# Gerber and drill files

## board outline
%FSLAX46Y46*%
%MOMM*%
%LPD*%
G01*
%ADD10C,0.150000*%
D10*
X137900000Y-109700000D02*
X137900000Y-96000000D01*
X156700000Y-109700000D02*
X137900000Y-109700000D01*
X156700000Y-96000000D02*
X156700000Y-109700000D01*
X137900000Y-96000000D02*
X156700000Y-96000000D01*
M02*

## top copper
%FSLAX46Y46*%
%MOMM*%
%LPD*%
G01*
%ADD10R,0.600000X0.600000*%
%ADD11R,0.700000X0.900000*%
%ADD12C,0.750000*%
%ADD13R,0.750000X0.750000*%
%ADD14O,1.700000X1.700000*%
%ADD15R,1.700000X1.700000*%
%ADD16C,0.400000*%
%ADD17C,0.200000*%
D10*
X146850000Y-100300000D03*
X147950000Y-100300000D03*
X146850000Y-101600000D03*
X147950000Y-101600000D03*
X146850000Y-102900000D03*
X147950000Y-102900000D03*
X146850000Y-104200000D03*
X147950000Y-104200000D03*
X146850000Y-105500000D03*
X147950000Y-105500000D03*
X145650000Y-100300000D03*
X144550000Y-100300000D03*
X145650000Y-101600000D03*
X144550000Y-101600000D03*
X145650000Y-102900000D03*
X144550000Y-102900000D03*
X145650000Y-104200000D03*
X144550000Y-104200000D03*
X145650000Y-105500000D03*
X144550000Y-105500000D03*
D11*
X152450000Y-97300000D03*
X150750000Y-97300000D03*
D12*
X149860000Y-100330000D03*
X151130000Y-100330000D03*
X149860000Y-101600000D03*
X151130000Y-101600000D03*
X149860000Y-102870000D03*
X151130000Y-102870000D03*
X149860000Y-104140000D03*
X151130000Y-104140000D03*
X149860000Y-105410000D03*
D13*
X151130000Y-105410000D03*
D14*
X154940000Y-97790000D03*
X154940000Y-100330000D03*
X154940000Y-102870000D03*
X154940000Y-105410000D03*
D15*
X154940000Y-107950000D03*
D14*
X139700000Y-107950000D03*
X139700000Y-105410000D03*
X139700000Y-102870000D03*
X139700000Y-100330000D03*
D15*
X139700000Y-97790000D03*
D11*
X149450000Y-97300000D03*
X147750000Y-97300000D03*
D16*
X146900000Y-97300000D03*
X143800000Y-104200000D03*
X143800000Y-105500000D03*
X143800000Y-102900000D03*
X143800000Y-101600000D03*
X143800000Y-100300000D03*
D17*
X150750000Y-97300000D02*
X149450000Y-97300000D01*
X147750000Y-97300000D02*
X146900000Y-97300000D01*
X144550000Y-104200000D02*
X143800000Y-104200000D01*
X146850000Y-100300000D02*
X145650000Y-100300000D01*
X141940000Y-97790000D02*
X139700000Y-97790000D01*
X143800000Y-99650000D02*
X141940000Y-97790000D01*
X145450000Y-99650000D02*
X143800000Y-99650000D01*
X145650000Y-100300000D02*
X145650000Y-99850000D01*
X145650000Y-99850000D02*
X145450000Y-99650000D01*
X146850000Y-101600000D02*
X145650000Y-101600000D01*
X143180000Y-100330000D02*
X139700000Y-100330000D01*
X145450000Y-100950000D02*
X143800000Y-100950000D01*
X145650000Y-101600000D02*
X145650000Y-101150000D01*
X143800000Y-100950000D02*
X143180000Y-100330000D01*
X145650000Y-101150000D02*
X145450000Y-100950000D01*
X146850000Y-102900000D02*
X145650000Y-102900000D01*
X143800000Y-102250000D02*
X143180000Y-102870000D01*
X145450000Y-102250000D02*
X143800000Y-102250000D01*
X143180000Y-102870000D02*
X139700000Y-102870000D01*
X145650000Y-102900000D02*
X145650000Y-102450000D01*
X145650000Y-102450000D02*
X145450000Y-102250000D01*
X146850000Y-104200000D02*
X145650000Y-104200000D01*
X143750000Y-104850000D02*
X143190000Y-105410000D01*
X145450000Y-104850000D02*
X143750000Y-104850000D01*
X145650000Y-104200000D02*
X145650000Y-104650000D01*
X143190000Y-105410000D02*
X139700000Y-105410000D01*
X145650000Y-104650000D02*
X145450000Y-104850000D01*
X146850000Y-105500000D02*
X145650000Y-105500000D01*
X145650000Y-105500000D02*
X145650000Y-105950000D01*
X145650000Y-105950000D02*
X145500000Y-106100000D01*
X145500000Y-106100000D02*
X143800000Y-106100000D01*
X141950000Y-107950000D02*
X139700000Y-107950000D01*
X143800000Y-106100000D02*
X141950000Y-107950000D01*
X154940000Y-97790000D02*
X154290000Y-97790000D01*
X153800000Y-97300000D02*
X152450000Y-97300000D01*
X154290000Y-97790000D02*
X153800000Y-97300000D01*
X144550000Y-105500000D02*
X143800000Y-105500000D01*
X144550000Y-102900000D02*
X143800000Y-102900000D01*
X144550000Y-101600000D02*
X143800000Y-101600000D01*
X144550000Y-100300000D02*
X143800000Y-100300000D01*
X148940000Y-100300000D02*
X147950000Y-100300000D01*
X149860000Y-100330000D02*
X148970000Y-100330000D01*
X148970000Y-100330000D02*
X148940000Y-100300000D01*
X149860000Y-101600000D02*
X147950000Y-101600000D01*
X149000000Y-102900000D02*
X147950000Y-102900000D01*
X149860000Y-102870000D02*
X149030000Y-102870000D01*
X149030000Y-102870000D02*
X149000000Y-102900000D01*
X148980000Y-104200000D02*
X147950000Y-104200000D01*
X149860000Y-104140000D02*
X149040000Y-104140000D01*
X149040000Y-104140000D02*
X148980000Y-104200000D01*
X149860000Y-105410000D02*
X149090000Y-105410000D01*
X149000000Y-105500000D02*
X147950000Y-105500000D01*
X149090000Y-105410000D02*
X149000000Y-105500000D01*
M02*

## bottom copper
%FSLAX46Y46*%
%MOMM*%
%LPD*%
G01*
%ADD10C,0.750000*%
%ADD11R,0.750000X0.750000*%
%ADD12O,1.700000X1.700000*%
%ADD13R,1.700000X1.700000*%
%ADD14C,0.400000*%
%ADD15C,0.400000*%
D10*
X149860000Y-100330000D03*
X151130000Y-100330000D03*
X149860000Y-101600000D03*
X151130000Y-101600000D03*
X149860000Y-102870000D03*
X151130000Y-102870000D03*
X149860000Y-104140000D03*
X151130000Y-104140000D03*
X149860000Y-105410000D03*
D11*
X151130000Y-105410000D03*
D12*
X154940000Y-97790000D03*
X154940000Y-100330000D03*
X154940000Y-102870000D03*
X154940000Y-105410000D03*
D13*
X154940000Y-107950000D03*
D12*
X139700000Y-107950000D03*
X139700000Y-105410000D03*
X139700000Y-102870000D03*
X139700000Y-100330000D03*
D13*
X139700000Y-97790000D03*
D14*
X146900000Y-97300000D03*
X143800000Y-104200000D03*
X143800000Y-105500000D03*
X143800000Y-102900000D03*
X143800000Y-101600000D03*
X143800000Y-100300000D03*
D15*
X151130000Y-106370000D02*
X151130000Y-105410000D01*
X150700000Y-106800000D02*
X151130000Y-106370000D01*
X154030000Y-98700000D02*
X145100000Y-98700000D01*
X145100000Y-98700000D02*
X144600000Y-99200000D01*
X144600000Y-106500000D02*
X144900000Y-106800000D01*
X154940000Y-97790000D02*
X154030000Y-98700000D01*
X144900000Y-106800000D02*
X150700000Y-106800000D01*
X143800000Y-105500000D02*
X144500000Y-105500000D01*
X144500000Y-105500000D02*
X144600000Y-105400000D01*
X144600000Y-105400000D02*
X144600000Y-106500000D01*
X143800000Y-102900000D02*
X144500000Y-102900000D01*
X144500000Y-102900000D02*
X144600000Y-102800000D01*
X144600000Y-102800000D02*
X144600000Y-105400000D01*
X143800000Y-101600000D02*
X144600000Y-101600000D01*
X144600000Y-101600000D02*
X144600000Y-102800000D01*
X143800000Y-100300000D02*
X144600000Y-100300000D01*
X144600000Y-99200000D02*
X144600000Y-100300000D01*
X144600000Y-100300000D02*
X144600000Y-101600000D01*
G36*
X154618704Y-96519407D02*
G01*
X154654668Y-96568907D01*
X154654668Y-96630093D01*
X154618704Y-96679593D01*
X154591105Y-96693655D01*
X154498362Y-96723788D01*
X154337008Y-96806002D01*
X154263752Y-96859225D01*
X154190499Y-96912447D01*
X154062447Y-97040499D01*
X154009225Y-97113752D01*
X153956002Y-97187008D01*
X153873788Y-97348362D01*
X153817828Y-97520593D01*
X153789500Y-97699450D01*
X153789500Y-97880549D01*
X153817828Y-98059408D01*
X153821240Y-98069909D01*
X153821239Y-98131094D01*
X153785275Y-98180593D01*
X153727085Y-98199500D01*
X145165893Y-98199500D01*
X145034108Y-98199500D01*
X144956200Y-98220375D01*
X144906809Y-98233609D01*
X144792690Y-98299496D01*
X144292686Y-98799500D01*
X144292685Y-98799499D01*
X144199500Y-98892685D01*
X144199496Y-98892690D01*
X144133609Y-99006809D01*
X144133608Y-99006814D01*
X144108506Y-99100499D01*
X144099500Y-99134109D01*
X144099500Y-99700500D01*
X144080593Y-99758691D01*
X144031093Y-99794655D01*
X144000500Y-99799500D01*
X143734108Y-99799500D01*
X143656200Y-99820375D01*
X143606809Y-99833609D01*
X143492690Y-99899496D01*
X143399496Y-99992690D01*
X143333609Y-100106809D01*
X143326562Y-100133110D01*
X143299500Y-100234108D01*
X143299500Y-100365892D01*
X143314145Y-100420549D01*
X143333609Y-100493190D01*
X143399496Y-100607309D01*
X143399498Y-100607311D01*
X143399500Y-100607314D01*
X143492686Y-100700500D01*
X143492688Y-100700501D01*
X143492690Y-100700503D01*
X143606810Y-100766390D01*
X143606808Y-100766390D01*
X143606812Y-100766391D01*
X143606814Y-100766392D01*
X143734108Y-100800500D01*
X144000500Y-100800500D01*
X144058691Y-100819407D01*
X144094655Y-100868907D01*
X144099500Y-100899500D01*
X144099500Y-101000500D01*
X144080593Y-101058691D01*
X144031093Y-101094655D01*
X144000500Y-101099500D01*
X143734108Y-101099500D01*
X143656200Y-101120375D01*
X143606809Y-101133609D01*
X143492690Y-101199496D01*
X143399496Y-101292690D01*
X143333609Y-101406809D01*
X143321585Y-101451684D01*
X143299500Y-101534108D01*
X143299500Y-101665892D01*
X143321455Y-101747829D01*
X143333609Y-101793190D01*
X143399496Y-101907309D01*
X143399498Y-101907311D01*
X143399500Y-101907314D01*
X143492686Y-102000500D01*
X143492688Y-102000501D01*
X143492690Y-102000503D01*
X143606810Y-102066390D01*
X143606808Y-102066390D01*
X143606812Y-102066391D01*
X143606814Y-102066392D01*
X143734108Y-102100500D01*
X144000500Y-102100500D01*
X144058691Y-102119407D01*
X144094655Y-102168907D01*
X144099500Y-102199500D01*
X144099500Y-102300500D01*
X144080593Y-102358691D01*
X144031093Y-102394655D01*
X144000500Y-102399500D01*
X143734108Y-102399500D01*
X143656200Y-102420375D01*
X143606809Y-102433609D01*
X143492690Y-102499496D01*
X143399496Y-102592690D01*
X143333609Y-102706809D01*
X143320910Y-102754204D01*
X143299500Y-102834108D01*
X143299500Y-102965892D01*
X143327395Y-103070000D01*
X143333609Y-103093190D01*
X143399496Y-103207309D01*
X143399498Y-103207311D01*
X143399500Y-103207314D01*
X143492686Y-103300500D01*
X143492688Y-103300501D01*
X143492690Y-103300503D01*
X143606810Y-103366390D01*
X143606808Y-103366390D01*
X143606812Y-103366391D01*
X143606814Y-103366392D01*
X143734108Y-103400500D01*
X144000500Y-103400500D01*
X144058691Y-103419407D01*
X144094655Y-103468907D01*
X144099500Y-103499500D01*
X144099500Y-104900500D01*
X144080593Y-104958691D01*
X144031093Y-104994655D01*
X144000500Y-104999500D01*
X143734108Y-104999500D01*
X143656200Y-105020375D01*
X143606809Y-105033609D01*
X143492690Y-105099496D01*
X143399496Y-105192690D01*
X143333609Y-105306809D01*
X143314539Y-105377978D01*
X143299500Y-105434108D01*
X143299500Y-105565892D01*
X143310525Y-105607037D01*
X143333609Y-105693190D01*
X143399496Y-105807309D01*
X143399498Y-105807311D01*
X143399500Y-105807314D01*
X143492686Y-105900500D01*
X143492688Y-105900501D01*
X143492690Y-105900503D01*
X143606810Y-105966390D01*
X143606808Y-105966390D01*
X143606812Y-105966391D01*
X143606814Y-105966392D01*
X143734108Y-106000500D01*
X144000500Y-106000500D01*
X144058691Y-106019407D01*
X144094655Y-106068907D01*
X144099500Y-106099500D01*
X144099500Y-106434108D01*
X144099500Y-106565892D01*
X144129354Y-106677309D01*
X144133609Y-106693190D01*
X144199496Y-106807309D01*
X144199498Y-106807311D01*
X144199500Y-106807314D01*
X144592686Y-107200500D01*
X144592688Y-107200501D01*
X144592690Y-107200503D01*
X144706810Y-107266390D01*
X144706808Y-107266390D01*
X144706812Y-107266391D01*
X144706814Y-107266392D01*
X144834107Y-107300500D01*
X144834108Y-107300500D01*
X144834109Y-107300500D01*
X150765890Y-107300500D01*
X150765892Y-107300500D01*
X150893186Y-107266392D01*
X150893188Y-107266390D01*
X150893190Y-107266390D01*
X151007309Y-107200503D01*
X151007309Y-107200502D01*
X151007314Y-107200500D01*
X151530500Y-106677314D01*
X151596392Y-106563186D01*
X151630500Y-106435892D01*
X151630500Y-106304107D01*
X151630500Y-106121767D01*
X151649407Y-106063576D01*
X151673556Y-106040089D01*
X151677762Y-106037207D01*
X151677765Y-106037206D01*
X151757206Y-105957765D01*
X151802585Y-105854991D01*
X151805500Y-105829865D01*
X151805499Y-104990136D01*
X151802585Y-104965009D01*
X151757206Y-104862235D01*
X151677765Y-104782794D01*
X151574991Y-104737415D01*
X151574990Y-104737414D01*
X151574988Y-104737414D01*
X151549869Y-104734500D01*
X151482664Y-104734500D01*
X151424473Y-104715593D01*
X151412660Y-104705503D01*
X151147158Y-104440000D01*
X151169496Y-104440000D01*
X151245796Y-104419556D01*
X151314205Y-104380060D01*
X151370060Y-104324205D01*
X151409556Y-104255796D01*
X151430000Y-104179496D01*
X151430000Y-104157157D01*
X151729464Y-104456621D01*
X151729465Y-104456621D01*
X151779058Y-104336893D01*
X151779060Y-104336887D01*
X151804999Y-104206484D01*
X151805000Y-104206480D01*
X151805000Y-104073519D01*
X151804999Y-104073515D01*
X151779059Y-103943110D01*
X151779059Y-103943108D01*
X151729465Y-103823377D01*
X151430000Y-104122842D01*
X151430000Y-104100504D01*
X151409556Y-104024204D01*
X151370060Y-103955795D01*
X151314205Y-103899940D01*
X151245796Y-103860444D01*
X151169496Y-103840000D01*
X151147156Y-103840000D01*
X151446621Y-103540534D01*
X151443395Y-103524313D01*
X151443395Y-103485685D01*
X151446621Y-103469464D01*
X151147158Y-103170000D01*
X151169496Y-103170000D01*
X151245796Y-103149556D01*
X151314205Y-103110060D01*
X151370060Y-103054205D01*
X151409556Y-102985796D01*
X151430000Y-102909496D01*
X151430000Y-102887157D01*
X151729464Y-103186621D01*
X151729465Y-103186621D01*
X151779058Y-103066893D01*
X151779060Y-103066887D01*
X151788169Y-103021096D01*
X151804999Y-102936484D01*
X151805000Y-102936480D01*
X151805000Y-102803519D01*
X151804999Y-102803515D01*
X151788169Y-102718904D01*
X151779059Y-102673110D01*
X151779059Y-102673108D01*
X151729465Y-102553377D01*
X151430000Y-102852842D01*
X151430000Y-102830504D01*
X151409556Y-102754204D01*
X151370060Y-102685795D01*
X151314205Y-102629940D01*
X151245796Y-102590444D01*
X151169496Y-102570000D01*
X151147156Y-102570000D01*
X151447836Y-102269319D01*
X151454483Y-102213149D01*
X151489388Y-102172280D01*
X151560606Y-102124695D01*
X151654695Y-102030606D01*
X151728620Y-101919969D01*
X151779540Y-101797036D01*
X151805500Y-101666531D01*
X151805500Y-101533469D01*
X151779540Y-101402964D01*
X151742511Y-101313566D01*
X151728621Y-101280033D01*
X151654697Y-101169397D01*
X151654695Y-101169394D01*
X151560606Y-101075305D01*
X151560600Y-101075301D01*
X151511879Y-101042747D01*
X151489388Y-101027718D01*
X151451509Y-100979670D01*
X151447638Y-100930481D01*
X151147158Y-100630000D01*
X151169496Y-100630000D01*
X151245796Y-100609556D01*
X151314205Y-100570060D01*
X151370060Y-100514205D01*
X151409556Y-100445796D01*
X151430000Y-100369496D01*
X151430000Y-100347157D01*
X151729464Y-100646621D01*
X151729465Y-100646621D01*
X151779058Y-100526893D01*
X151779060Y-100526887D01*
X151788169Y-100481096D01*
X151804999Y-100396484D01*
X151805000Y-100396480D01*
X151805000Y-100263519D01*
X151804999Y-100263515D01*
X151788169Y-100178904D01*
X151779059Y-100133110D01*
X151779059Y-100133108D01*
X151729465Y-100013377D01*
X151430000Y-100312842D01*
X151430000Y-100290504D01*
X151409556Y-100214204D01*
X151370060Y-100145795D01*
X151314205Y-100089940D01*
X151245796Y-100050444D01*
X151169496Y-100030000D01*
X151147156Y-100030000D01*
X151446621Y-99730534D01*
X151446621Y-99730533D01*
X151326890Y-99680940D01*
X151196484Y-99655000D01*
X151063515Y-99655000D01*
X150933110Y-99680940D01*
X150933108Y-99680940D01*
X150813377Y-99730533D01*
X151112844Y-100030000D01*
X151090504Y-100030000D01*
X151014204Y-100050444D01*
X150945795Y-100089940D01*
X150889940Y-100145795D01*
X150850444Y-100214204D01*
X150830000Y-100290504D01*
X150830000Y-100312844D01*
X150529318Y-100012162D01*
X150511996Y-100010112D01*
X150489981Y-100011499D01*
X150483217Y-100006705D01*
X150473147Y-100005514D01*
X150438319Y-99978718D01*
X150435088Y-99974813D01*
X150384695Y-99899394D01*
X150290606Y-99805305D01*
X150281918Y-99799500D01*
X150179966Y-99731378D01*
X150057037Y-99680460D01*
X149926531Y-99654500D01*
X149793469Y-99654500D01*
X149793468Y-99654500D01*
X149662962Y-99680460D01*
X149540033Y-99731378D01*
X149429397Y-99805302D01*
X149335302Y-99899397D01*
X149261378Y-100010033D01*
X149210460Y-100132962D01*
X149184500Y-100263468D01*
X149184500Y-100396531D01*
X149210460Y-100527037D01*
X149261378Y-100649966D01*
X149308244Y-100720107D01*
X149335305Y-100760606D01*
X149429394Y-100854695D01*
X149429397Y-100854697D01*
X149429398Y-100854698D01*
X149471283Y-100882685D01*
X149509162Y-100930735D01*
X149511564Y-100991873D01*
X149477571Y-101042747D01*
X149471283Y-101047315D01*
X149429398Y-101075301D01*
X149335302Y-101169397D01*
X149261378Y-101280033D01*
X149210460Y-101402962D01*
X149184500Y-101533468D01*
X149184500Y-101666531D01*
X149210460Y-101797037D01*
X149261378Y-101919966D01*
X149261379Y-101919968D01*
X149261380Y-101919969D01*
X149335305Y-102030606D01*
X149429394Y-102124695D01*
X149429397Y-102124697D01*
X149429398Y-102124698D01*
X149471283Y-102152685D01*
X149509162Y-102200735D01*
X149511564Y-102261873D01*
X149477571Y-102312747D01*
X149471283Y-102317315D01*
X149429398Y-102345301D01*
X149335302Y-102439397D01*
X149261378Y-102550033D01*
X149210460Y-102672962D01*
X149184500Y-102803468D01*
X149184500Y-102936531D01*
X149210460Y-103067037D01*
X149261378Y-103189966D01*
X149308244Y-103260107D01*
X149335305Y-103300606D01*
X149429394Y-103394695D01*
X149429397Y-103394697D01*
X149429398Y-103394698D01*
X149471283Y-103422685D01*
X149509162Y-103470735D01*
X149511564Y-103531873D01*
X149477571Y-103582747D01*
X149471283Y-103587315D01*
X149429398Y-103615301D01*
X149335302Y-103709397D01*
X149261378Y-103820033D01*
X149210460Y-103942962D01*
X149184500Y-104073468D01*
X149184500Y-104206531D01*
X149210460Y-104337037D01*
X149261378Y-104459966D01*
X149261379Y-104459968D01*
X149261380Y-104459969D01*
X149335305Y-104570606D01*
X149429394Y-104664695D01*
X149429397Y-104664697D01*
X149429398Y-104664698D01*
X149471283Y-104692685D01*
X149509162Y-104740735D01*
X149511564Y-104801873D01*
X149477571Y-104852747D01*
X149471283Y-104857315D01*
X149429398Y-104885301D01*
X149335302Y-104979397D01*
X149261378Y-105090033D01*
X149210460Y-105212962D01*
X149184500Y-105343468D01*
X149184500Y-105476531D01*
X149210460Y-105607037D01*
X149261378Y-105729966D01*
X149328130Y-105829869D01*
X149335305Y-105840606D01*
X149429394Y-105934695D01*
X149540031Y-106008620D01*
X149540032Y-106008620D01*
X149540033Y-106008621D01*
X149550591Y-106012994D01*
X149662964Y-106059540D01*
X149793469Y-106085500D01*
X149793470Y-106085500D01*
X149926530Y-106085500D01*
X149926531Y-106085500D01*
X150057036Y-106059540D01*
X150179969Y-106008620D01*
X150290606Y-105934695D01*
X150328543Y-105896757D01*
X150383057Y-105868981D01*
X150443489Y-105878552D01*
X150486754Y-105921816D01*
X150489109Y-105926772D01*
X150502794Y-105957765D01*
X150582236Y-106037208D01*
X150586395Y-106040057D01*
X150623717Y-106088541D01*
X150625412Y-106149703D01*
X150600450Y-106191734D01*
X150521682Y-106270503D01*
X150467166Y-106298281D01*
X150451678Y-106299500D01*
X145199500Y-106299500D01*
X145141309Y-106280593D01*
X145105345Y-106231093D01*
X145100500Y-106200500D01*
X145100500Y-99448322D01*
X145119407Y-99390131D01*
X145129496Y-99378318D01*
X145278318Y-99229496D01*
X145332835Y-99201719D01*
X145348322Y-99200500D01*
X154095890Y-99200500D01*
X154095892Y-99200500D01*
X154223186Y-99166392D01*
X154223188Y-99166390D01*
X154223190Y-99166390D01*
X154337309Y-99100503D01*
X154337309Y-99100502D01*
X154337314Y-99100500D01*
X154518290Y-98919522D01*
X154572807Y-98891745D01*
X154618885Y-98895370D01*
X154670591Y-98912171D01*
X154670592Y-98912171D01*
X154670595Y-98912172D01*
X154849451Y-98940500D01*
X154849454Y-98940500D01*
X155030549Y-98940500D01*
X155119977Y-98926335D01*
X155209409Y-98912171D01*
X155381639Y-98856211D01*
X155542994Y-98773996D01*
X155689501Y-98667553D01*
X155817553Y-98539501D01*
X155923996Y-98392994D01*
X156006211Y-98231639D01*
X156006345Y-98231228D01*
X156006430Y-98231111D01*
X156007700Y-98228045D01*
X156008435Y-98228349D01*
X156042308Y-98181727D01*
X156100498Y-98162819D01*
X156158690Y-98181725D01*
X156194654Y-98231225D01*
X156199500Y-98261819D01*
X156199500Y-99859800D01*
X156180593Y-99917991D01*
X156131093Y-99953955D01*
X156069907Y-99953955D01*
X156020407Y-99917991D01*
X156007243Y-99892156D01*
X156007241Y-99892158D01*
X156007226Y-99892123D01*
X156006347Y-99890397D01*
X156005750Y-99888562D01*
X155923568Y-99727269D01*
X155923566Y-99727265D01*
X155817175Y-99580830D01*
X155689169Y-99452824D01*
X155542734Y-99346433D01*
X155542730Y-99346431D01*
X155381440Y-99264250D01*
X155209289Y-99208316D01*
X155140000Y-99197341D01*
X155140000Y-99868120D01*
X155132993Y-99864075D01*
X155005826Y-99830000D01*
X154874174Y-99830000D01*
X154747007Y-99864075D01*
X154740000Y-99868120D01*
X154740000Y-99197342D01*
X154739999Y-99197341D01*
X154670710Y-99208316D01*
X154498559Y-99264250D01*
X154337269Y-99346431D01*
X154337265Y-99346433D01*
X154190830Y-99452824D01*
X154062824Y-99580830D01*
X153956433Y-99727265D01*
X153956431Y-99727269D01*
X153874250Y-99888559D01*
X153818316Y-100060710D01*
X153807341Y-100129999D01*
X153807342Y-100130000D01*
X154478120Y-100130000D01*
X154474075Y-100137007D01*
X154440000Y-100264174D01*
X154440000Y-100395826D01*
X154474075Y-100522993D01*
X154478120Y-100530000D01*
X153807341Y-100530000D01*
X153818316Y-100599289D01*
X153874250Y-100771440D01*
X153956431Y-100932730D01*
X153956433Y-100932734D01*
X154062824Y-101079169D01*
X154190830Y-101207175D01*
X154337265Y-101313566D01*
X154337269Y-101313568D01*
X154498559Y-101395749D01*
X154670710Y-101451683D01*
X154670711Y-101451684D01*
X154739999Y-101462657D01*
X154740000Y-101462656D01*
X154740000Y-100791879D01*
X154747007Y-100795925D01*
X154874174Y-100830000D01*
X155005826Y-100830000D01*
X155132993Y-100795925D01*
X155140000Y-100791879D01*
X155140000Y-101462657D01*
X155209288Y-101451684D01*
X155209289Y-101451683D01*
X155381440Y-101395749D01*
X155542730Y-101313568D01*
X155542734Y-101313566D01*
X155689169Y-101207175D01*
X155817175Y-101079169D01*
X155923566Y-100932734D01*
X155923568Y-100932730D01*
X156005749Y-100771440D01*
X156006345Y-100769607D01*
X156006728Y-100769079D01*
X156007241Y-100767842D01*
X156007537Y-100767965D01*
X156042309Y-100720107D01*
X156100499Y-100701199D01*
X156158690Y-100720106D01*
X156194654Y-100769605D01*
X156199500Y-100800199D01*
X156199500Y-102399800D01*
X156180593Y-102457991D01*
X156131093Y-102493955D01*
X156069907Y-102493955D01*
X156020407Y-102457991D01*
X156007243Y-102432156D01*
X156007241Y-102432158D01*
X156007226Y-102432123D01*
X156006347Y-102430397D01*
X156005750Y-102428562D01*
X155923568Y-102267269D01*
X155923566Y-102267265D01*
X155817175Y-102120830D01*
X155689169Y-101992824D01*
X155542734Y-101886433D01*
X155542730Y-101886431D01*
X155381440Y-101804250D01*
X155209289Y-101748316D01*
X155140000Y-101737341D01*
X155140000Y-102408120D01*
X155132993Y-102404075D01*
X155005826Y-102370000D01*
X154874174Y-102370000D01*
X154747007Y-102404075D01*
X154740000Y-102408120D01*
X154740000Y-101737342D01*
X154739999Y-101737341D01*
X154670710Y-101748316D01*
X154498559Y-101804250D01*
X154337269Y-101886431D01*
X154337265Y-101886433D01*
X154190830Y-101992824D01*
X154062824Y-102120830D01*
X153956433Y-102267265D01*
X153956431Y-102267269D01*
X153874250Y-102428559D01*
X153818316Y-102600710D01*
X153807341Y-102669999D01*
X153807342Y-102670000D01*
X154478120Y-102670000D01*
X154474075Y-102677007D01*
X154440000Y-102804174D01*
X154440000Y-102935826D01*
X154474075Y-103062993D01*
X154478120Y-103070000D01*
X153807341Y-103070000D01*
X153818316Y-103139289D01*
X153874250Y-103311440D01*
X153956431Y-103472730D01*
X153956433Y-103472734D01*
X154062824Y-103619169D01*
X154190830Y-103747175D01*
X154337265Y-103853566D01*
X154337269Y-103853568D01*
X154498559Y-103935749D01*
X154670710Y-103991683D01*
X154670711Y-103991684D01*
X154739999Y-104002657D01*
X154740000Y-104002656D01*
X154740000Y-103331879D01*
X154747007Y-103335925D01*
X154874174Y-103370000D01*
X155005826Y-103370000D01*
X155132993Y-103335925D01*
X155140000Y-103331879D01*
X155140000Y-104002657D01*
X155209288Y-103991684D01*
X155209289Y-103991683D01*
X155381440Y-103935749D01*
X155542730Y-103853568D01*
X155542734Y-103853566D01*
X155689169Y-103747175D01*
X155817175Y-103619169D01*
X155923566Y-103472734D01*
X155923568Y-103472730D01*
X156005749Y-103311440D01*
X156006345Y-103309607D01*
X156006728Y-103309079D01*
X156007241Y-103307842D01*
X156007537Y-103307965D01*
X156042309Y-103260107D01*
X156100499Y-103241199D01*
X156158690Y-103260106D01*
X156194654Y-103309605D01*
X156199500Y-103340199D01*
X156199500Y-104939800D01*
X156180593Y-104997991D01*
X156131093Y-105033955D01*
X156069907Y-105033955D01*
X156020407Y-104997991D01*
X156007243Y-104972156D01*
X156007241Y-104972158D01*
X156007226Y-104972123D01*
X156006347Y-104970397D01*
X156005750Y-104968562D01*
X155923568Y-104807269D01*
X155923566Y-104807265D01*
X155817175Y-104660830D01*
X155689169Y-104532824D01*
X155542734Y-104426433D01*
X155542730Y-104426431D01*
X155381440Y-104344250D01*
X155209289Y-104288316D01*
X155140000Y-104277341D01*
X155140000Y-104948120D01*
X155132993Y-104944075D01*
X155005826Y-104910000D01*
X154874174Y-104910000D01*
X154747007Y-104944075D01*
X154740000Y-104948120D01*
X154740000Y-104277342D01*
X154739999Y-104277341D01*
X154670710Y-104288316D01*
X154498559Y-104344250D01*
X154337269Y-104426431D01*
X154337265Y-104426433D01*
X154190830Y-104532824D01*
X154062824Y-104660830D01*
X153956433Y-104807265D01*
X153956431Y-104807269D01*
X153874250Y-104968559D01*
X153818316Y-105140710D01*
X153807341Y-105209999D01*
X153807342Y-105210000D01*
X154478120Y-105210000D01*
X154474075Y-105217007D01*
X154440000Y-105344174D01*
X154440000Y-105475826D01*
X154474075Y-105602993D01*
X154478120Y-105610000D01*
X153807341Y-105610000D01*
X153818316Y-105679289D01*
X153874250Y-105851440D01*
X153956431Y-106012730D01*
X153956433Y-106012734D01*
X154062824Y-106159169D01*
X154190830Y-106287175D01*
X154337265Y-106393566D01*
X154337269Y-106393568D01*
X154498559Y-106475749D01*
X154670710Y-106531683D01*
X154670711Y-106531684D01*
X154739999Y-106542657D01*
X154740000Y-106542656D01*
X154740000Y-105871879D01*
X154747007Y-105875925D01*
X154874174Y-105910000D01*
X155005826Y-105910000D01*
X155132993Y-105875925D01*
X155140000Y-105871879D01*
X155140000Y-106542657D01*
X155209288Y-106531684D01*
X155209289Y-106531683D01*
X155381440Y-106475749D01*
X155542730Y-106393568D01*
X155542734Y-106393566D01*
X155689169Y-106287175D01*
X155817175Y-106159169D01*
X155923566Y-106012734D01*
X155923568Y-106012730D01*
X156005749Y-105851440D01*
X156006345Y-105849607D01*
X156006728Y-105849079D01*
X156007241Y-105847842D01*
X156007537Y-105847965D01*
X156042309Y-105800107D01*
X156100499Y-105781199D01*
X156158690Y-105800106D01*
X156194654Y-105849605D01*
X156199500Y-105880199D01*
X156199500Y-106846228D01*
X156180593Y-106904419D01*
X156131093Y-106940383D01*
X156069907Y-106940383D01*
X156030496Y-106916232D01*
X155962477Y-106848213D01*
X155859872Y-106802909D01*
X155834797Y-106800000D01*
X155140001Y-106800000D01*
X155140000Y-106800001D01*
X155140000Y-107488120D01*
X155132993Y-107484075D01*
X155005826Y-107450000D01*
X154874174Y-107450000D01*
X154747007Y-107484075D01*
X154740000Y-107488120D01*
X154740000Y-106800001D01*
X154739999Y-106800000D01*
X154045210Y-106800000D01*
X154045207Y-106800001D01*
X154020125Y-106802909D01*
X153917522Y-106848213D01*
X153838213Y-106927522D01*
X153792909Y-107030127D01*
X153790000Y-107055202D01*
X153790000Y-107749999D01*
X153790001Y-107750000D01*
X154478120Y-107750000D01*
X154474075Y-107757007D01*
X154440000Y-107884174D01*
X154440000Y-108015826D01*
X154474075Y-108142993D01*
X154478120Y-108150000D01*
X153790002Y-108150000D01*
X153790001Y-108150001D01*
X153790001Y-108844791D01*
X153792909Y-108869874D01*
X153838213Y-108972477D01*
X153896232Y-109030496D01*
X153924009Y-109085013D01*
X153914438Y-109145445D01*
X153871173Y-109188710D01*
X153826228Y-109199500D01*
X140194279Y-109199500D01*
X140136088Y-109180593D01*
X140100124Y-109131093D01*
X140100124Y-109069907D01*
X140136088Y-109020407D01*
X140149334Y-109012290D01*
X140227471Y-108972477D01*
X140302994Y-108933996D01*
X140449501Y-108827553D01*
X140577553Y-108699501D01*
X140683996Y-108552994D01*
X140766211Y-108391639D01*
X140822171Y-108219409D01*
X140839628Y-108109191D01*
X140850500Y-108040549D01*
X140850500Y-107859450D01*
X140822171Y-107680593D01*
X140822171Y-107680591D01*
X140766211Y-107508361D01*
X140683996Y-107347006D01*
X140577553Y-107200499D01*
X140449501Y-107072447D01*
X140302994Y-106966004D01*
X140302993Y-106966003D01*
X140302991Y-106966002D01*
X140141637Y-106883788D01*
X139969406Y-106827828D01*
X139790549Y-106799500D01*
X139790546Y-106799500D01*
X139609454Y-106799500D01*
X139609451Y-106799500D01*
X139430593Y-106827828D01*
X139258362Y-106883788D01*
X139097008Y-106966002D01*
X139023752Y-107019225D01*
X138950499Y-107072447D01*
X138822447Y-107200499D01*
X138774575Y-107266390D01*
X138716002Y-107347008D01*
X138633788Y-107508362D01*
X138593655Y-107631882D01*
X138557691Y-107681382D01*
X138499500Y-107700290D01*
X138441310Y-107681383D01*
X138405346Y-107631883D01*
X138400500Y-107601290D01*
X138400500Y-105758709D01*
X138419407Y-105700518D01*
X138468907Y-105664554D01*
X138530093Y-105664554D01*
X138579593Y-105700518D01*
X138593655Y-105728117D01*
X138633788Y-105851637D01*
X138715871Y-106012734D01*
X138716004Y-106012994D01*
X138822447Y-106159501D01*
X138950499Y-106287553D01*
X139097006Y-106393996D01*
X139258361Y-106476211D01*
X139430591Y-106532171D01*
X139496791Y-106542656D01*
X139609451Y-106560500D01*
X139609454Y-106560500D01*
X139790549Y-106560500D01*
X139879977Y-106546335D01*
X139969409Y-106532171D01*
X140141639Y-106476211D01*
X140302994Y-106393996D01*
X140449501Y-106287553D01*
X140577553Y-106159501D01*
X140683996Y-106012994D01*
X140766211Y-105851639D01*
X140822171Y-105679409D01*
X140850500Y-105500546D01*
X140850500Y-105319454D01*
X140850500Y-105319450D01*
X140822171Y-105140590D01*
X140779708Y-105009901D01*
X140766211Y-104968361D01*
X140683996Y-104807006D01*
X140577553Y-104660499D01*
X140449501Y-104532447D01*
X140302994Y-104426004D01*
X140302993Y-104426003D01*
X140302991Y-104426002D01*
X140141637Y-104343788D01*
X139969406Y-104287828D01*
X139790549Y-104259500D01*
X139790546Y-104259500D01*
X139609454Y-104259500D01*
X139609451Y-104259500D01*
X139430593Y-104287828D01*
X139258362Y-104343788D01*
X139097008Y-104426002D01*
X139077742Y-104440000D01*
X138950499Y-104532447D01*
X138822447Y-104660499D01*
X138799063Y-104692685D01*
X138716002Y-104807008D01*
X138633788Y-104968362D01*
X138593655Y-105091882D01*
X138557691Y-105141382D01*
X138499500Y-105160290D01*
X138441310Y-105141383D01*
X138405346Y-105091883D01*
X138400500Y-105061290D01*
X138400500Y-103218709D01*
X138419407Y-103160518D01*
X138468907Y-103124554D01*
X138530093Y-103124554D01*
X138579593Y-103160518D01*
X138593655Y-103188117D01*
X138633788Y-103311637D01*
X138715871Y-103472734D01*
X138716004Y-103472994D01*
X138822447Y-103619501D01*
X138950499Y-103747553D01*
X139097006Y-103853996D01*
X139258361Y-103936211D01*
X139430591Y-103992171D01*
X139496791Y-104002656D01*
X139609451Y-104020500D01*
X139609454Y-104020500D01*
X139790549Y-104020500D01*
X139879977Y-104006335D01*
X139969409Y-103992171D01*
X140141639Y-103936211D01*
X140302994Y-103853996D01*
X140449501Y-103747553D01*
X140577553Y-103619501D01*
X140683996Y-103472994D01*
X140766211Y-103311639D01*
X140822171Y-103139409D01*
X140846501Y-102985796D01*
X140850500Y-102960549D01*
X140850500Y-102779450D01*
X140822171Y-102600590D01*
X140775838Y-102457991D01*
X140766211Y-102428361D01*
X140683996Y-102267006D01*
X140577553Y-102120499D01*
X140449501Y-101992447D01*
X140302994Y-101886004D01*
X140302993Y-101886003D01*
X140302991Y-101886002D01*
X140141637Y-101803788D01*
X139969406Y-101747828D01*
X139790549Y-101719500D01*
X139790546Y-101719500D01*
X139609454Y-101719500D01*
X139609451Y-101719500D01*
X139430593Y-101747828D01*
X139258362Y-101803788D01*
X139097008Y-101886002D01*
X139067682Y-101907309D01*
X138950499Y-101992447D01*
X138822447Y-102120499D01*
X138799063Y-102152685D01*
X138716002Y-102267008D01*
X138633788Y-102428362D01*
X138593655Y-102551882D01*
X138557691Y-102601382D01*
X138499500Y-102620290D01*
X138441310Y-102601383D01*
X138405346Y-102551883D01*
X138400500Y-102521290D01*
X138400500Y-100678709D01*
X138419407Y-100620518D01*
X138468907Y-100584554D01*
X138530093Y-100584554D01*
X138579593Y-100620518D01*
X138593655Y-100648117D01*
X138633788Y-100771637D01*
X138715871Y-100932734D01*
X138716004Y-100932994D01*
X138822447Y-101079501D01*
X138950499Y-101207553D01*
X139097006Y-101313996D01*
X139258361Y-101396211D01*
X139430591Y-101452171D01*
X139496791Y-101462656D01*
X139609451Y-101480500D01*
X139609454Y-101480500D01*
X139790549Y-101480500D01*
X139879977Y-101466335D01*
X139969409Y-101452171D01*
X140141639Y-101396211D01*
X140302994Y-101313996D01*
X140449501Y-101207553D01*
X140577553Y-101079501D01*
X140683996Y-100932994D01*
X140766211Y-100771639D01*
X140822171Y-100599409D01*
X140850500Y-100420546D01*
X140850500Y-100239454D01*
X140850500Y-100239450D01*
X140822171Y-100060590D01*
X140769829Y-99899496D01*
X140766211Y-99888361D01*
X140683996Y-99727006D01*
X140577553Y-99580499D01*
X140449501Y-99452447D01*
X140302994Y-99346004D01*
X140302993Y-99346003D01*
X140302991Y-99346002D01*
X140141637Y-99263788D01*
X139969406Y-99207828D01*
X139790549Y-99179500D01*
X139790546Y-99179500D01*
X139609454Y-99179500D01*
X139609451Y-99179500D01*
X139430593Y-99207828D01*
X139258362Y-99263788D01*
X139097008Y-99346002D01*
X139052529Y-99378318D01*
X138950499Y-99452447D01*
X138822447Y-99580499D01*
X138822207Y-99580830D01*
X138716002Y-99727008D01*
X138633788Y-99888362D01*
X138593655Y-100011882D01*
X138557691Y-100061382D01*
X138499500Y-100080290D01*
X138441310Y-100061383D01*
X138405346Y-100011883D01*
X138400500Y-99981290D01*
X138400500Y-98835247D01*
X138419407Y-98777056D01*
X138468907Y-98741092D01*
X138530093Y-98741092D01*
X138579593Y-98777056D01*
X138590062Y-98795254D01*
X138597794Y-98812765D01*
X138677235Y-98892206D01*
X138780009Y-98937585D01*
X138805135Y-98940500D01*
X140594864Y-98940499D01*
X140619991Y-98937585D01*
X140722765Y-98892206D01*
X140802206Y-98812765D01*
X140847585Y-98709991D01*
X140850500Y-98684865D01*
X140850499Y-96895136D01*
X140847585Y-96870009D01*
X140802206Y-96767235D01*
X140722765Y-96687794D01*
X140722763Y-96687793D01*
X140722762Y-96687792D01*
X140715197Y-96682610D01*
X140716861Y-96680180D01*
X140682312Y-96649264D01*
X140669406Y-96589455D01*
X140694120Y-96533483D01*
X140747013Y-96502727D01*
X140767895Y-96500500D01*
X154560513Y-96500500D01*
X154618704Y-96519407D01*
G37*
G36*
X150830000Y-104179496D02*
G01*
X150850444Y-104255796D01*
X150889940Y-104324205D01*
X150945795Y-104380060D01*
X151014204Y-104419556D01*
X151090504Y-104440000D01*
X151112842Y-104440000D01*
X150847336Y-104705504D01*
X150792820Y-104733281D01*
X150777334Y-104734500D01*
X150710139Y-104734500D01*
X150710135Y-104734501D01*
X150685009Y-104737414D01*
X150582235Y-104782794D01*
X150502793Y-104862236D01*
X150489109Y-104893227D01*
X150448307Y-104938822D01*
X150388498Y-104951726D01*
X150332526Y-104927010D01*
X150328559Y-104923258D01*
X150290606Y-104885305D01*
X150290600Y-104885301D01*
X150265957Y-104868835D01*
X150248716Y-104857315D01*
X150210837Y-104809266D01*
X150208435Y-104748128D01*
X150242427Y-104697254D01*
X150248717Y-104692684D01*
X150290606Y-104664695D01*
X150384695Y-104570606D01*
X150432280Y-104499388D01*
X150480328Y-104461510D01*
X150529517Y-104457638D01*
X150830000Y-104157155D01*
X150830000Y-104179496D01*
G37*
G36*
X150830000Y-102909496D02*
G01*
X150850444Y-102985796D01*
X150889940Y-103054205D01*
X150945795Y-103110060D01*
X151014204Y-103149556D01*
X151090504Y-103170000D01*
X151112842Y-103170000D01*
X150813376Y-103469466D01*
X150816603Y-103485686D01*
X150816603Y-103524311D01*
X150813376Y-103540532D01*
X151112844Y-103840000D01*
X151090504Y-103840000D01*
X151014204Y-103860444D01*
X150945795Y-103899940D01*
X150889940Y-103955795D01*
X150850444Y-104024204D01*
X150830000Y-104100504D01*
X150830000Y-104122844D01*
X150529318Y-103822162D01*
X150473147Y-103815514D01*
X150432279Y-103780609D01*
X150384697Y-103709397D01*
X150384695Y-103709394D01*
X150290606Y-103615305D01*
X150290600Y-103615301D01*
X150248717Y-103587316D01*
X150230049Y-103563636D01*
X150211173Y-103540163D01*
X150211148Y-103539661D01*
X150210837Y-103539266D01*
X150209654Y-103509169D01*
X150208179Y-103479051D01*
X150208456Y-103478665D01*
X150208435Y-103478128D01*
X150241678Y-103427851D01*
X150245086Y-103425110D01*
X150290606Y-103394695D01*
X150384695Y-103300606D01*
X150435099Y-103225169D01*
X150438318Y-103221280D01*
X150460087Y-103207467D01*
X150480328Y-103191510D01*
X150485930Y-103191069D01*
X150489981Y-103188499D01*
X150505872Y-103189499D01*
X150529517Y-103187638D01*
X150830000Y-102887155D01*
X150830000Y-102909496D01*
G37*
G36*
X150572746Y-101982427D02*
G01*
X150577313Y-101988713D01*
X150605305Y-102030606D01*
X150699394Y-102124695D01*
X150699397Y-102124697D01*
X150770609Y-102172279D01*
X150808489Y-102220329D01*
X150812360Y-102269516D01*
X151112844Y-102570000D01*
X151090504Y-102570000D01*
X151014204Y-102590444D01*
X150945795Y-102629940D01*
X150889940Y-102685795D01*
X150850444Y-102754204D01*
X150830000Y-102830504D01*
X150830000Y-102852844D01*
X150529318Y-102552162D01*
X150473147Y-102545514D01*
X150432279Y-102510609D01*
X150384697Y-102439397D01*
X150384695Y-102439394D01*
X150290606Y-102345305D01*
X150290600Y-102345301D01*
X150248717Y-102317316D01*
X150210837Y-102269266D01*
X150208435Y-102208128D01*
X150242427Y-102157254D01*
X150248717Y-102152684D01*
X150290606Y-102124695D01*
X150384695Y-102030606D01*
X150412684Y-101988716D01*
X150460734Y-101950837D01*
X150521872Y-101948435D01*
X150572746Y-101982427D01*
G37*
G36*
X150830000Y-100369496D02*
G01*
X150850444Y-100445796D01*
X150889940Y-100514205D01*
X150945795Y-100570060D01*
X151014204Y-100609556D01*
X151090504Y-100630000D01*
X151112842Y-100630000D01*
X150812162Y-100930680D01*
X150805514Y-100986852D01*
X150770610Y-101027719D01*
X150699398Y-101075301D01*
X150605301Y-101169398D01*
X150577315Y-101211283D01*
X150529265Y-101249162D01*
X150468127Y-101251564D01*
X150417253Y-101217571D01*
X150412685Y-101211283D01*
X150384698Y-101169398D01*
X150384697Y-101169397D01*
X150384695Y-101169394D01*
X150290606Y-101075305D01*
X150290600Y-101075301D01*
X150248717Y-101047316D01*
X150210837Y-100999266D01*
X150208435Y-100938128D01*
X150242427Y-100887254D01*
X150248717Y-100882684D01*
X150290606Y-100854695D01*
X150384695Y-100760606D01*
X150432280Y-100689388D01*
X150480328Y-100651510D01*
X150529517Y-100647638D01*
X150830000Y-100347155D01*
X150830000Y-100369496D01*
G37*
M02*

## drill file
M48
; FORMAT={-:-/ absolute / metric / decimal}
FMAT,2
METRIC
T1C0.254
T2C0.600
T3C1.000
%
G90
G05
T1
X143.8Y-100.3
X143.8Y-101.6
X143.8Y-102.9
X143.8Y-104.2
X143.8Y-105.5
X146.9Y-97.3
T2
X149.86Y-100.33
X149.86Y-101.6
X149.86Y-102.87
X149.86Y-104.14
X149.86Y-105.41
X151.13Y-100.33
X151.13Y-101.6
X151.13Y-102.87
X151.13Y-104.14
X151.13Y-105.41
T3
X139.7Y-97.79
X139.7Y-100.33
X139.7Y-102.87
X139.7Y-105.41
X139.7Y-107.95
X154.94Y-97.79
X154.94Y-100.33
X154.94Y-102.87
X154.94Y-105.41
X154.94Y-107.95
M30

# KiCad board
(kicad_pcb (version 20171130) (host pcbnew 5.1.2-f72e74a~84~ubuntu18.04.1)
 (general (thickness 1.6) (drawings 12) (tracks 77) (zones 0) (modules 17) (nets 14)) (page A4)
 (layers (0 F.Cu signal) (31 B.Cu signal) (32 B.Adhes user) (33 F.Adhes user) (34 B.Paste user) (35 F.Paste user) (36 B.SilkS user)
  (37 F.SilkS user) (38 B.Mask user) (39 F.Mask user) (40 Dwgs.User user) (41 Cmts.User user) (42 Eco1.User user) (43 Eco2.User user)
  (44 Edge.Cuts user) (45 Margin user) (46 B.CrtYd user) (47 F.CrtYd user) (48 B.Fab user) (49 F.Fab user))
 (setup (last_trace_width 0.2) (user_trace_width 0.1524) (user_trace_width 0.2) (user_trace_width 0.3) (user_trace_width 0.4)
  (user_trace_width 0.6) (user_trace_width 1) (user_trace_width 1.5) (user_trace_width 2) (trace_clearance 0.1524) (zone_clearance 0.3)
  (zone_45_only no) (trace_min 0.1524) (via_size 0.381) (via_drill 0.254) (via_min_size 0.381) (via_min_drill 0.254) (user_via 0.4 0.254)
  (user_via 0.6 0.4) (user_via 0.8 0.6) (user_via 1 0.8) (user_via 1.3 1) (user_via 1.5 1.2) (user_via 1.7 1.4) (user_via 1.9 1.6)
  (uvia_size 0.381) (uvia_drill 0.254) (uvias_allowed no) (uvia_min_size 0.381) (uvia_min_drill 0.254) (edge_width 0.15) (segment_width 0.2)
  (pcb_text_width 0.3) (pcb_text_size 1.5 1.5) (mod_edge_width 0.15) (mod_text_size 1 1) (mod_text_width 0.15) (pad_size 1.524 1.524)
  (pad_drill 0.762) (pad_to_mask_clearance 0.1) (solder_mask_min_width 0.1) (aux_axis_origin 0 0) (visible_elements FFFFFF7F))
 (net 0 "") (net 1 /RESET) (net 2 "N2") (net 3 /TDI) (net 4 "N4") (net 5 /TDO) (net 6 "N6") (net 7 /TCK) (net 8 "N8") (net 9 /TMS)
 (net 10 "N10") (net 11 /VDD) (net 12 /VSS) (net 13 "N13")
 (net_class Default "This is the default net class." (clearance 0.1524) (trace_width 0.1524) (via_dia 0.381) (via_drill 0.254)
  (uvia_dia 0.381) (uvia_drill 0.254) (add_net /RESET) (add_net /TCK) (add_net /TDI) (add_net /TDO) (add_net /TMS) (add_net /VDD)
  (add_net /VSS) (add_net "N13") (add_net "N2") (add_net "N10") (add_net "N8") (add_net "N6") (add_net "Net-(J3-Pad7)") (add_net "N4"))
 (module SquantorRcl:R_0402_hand (layer F.Cu) (at 147.4 100.3 180)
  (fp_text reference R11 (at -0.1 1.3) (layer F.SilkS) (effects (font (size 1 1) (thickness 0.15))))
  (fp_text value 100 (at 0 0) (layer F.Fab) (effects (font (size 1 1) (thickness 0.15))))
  (pad 2 smd rect (at 0.55 0 180) (size 0.6 0.6) (layers F.Cu F.Paste F.Mask) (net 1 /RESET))
  (pad 1 smd rect (at -0.55 0 180) (size 0.6 0.6) (layers F.Cu F.Paste F.Mask) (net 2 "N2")))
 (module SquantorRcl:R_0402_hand (layer F.Cu) (at 147.4 101.6 180)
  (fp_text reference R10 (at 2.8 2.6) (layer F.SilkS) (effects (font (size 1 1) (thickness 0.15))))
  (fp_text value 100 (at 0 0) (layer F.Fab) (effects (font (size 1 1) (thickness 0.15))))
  (pad 2 smd rect (at 0.55 0 180) (size 0.6 0.6) (layers F.Cu F.Paste F.Mask) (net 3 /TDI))
  (pad 1 smd rect (at -0.55 0 180) (size 0.6 0.6) (layers F.Cu F.Paste F.Mask) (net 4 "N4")))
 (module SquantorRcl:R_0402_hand (layer F.Cu) (at 147.4 102.9 180)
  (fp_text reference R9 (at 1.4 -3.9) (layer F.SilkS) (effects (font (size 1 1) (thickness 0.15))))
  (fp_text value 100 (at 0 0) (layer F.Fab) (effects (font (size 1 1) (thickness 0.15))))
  (pad 2 smd rect (at 0.55 0 180) (size 0.6 0.6) (layers F.Cu F.Paste F.Mask) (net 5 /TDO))
  (pad 1 smd rect (at -0.55 0 180) (size 0.6 0.6) (layers F.Cu F.Paste F.Mask) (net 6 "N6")))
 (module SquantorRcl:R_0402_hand (layer F.Cu) (at 147.4 104.2 180)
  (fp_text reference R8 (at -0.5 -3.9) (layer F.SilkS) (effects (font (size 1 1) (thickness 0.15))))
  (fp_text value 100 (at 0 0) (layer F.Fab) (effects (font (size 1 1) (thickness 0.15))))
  (pad 2 smd rect (at 0.55 0 180) (size 0.6 0.6) (layers F.Cu F.Paste F.Mask) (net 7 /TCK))
  (pad 1 smd rect (at -0.55 0 180) (size 0.6 0.6) (layers F.Cu F.Paste F.Mask) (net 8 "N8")))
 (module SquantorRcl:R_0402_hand (layer F.Cu) (at 147.4 105.5 180)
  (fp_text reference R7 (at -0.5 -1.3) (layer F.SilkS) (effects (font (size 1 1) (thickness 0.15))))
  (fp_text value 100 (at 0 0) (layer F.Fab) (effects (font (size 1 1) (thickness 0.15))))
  (pad 2 smd rect (at 0.55 0 180) (size 0.6 0.6) (layers F.Cu F.Paste F.Mask) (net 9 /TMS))
  (pad 1 smd rect (at -0.55 0 180) (size 0.6 0.6) (layers F.Cu F.Paste F.Mask) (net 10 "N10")))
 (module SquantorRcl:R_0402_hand (layer F.Cu) (at 145.1 100.3)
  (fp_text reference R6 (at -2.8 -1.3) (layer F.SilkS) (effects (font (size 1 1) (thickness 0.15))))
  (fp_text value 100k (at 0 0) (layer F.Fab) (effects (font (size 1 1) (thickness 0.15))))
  (pad 2 smd rect (at 0.55 0) (size 0.6 0.6) (layers F.Cu F.Paste F.Mask) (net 1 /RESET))
  (pad 1 smd rect (at -0.55 0) (size 0.6 0.6) (layers F.Cu F.Paste F.Mask) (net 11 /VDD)))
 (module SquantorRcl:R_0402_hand (layer F.Cu) (at 145.1 101.6)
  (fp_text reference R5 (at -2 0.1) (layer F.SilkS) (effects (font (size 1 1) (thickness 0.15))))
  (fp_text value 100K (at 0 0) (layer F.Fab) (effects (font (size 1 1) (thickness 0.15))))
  (pad 2 smd rect (at 0.55 0) (size 0.6 0.6) (layers F.Cu F.Paste F.Mask) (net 3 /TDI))
  (pad 1 smd rect (at -0.55 0) (size 0.6 0.6) (layers F.Cu F.Paste F.Mask) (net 11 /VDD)))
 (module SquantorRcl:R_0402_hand (layer F.Cu) (at 145.1 102.9)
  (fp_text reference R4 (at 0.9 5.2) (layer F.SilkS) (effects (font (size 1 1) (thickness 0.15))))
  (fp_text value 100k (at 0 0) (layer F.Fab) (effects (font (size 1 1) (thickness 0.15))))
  (pad 2 smd rect (at 0.55 0) (size 0.6 0.6) (layers F.Cu F.Paste F.Mask) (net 5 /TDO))
  (pad 1 smd rect (at -0.55 0) (size 0.6 0.6) (layers F.Cu F.Paste F.Mask) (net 11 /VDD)))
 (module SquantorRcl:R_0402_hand (layer F.Cu) (at 145.1 104.2)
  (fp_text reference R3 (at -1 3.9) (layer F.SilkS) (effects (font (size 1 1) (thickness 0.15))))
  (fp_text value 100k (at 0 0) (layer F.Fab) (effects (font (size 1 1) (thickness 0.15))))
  (pad 2 smd rect (at 0.55 0) (size 0.6 0.6) (layers F.Cu F.Paste F.Mask) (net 7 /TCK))
  (pad 1 smd rect (at -0.55 0) (size 0.6 0.6) (layers F.Cu F.Paste F.Mask) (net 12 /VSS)))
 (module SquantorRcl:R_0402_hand (layer F.Cu) (at 145.1 105.5)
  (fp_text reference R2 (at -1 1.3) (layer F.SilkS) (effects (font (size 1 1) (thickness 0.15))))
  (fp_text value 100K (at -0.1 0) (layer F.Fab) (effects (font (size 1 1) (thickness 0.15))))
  (pad 2 smd rect (at 0.55 0) (size 0.6 0.6) (layers F.Cu F.Paste F.Mask) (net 9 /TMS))
  (pad 1 smd rect (at -0.55 0) (size 0.6 0.6) (layers F.Cu F.Paste F.Mask) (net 11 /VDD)))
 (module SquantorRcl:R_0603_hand (layer F.Cu) (at 151.6 97.3)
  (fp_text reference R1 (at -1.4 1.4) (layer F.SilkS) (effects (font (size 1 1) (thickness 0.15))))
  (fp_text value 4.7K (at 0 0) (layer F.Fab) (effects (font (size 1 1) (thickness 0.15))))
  (pad 2 smd rect (at 0.85 0) (size 0.7 0.9) (layers F.Cu F.Paste F.Mask) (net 11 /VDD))
  (pad 1 smd rect (at -0.85 0) (size 0.7 0.9) (layers F.Cu F.Paste F.Mask) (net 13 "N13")))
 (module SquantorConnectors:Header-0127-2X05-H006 (layer F.Cu) (at 150.495 102.87 90)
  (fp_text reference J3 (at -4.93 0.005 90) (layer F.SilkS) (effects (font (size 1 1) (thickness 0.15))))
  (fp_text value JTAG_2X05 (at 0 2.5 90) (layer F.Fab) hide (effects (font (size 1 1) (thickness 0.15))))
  (pad 10 thru_hole circle (at 2.54 -0.635 90) (size 0.75 0.75) (drill 0.6) (layers *.Cu *.Mask) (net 2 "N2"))
  (pad 9 thru_hole circle (at 2.54 0.635 90) (size 0.75 0.75) (drill 0.6) (layers *.Cu *.Mask) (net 12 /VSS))
  (pad 8 thru_hole circle (at 1.27 -0.635 90) (size 0.75 0.75) (drill 0.6) (layers *.Cu *.Mask) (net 4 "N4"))
  (pad 7 thru_hole circle (at 1.27 0.635 90) (size 0.75 0.75) (drill 0.6) (layers *.Cu *.Mask))
  (pad 6 thru_hole circle (at 0 -0.635 90) (size 0.75 0.75) (drill 0.6) (layers *.Cu *.Mask) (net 6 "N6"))
  (pad 5 thru_hole circle (at 0 0.635 90) (size 0.75 0.75) (drill 0.6) (layers *.Cu *.Mask) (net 12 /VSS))
  (pad 4 thru_hole circle (at -1.27 -0.635 90) (size 0.75 0.75) (drill 0.6) (layers *.Cu *.Mask) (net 8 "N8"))
  (pad 3 thru_hole circle (at -1.27 0.635 90) (size 0.75 0.75) (drill 0.6) (layers *.Cu *.Mask) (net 12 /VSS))
  (pad 2 thru_hole circle (at -2.54 -0.635 90) (size 0.75 0.75) (drill 0.6) (layers *.Cu *.Mask) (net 10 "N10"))
  (pad 1 thru_hole rect (at -2.54 0.635 90) (size 0.75 0.75) (drill 0.6) (layers *.Cu *.Mask) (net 11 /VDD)))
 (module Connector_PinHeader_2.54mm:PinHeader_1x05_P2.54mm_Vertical (layer B.Cu) (at 154.94 107.95)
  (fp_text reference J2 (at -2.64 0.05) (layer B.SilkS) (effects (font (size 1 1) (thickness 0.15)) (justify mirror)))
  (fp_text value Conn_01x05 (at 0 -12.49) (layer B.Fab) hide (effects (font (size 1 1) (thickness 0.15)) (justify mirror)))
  (pad 5 thru_hole oval (at 0 -10.16) (size 1.7 1.7) (drill 1) (layers *.Cu *.Mask) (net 11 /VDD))
  (pad 4 thru_hole oval (at 0 -7.62) (size 1.7 1.7) (drill 1) (layers *.Cu *.Mask) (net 12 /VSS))
  (pad 3 thru_hole oval (at 0 -5.08) (size 1.7 1.7) (drill 1) (layers *.Cu *.Mask) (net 12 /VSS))
  (pad 2 thru_hole oval (at 0 -2.54) (size 1.7 1.7) (drill 1) (layers *.Cu *.Mask) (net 12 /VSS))
  (pad 1 thru_hole rect (at 0 0) (size 1.7 1.7) (drill 1) (layers *.Cu *.Mask) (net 12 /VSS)))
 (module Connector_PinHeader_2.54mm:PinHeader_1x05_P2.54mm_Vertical (layer B.Cu) (at 139.7 97.79 180)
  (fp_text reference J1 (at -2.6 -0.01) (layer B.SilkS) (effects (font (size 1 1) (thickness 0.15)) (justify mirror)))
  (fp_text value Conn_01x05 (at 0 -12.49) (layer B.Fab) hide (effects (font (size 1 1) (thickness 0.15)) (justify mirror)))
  (pad 5 thru_hole oval (at 0 -10.16 180) (size 1.7 1.7) (drill 1) (layers *.Cu *.Mask) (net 9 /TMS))
  (pad 4 thru_hole oval (at 0 -7.62 180) (size 1.7 1.7) (drill 1) (layers *.Cu *.Mask) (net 7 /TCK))
  (pad 3 thru_hole oval (at 0 -5.08 180) (size 1.7 1.7) (drill 1) (layers *.Cu *.Mask) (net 5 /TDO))
  (pad 2 thru_hole oval (at 0 -2.54 180) (size 1.7 1.7) (drill 1) (layers *.Cu *.Mask) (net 3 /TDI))
  (pad 1 thru_hole rect (at 0 0 180) (size 1.7 1.7) (drill 1) (layers *.Cu *.Mask) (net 1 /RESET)))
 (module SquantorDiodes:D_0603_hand (layer F.Cu) (at 148.6 97.3)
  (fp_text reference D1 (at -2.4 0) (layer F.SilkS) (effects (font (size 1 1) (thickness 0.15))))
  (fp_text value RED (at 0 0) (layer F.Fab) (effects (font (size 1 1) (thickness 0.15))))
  (pad 2 smd rect (at 0.85 0) (size 0.7 0.9) (layers F.Cu F.Paste F.Mask) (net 13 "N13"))
  (pad 1 smd rect (at -0.85 0) (size 0.7 0.9) (layers F.Cu F.Paste F.Mask) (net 12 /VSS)))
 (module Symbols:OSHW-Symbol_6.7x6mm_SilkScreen (layer B.Cu) (at 145.9 103.4 180)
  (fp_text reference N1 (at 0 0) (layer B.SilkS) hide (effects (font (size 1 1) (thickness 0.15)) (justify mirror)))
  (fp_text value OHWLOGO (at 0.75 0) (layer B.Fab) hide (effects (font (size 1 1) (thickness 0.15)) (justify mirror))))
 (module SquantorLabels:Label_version (layer B.Cu) (at 145.9 107.2)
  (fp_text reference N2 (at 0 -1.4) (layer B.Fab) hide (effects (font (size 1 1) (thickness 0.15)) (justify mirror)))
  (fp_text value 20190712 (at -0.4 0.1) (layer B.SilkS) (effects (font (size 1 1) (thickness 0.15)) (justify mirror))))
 (gr_line (start 137.9 109.7) (end 137.9 96) (layer Edge.Cuts) (width 0.15))
 (gr_line (start 156.7 109.7) (end 137.9 109.7) (layer Edge.Cuts) (width 0.15))
 (gr_line (start 156.7 96) (end 156.7 109.7) (layer Edge.Cuts) (width 0.15))
 (gr_line (start 137.9 96) (end 156.7 96) (layer Edge.Cuts) (width 0.15))
 (segment (start 150.75 97.3) (end 149.45 97.3) (width 0.2) (layer F.Cu) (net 13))
 (via (at 146.9 97.3) (size 0.4) (drill 0.254) (layers F.Cu B.Cu) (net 12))
 (segment (start 147.75 97.3) (end 146.9 97.3) (width 0.2) (layer F.Cu) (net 12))
 (via (at 143.8 104.2) (size 0.4) (drill 0.254) (layers F.Cu B.Cu) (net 12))
 (segment (start 144.55 104.2) (end 143.8 104.2) (width 0.2) (layer F.Cu) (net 12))
 (segment (start 146.85 100.3) (end 145.65 100.3) (width 0.2) (layer F.Cu) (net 1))
 (segment (start 141.94 97.79) (end 139.7 97.79) (width 0.2) (layer F.Cu) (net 1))
 (segment (start 143.8 99.65) (end 141.94 97.79) (width 0.2) (layer F.Cu) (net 1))
 (segment (start 145.45 99.65) (end 143.8 99.65) (width 0.2) (layer F.Cu) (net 1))
 (segment (start 145.65 100.3) (end 145.65 99.85) (width 0.2) (layer F.Cu) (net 1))
 (segment (start 145.65 99.85) (end 145.45 99.65) (width 0.2) (layer F.Cu) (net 1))
 (segment (start 146.85 101.6) (end 145.65 101.6) (width 0.2) (layer F.Cu) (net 3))
 (segment (start 143.18 100.33) (end 139.7 100.33) (width 0.2) (layer F.Cu) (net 3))
 (segment (start 145.45 100.95) (end 143.8 100.95) (width 0.2) (layer F.Cu) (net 3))
 (segment (start 145.65 101.6) (end 145.65 101.15) (width 0.2) (layer F.Cu) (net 3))
 (segment (start 143.8 100.95) (end 143.18 100.33) (width 0.2) (layer F.Cu) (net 3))
 (segment (start 145.65 101.15) (end 145.45 100.95) (width 0.2) (layer F.Cu) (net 3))
 (segment (start 146.85 102.9) (end 145.65 102.9) (width 0.2) (layer F.Cu) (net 5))
 (segment (start 143.8 102.25) (end 143.18 102.87) (width 0.2) (layer F.Cu) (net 5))
 (segment (start 145.45 102.25) (end 143.8 102.25) (width 0.2) (layer F.Cu) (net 5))
 (segment (start 143.18 102.87) (end 139.7 102.87) (width 0.2) (layer F.Cu) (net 5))
 (segment (start 145.65 102.9) (end 145.65 102.45) (width 0.2) (layer F.Cu) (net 5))
 (segment (start 145.65 102.45) (end 145.45 102.25) (width 0.2) (layer F.Cu) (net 5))
 (segment (start 146.85 104.2) (end 145.65 104.2) (width 0.2) (layer F.Cu) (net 7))
 (segment (start 143.75 104.85) (end 143.19 105.41) (width 0.2) (layer F.Cu) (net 7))
 (segment (start 145.45 104.85) (end 143.75 104.85) (width 0.2) (layer F.Cu) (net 7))
 (segment (start 145.65 104.2) (end 145.65 104.65) (width 0.2) (layer F.Cu) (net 7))
 (segment (start 143.19 105.41) (end 139.7 105.41) (width 0.2) (layer F.Cu) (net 7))
 (segment (start 145.65 104.65) (end 145.45 104.85) (width 0.2) (layer F.Cu) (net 7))
 (segment (start 146.85 105.5) (end 145.65 105.5) (width 0.2) (layer F.Cu) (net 9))
 (segment (start 145.65 105.5) (end 145.65 105.95) (width 0.2) (layer F.Cu) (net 9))
 (segment (start 145.65 105.95) (end 145.5 106.1) (width 0.2) (layer F.Cu) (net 9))
 (segment (start 145.5 106.1) (end 143.8 106.1) (width 0.2) (layer F.Cu) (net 9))
 (segment (start 141.95 107.95) (end 139.7 107.95) (width 0.2) (layer F.Cu) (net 9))
 (segment (start 143.8 106.1) (end 141.95 107.95) (width 0.2) (layer F.Cu) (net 9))
 (segment (start 154.94 97.79) (end 154.29 97.79) (width 0.2) (layer F.Cu) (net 11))
 (segment (start 153.8 97.3) (end 152.45 97.3) (width 0.2) (layer F.Cu) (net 11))
 (segment (start 154.29 97.79) (end 153.8 97.3) (width 0.2) (layer F.Cu) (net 11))
 (via (at 143.8 105.5) (size 0.4) (drill 0.254) (layers F.Cu B.Cu) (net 11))
 (segment (start 144.55 105.5) (end 143.8 105.5) (width 0.2) (layer F.Cu) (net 11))
 (via (at 143.8 102.9) (size 0.4) (drill 0.254) (layers F.Cu B.Cu) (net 11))
 (segment (start 144.55 102.9) (end 143.8 102.9) (width 0.2) (layer F.Cu) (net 11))
 (via (at 143.8 101.6) (size 0.4) (drill 0.254) (layers F.Cu B.Cu) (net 11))
 (segment (start 144.55 101.6) (end 143.8 101.6) (width 0.2) (layer F.Cu) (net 11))
 (via (at 143.8 100.3) (size 0.4) (drill 0.254) (layers F.Cu B.Cu) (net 11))
 (segment (start 144.55 100.3) (end 143.8 100.3) (width 0.2) (layer F.Cu) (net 11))
 (segment (start 151.13 106.37) (end 151.13 105.41) (width 0.4) (layer B.Cu) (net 11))
 (segment (start 150.7 106.8) (end 151.13 106.37) (width 0.4) (layer B.Cu) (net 11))
 (segment (start 154.03 98.7) (end 145.1 98.7) (width 0.4) (layer B.Cu) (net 11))
 (segment (start 145.1 98.7) (end 144.6 99.2) (width 0.4) (layer B.Cu) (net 11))
 (segment (start 144.6 106.5) (end 144.9 106.8) (width 0.4) (layer B.Cu) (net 11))
 (segment (start 154.94 97.79) (end 154.03 98.7) (width 0.4) (layer B.Cu) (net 11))
 (segment (start 144.9 106.8) (end 150.7 106.8) (width 0.4) (layer B.Cu) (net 11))
 (segment (start 143.8 105.5) (end 144.5 105.5) (width 0.4) (layer B.Cu) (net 11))
 (segment (start 144.5 105.5) (end 144.6 105.4) (width 0.4) (layer B.Cu) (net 11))
 (segment (start 144.6 105.4) (end 144.6 106.5) (width 0.4) (layer B.Cu) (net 11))
 (segment (start 143.8 102.9) (end 144.5 102.9) (width 0.4) (layer B.Cu) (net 11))
 (segment (start 144.5 102.9) (end 144.6 102.8) (width 0.4) (layer B.Cu) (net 11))
 (segment (start 144.6 102.8) (end 144.6 105.4) (width 0.4) (layer B.Cu) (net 11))
 (segment (start 143.8 101.6) (end 144.6 101.6) (width 0.4) (layer B.Cu) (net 11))
 (segment (start 144.6 101.6) (end 144.6 102.8) (width 0.4) (layer B.Cu) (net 11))
 (segment (start 143.8 100.3) (end 144.6 100.3) (width 0.4) (layer B.Cu) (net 11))
 (segment (start 144.6 99.2) (end 144.6 100.3) (width 0.4) (layer B.Cu) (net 11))
 (segment (start 144.6 100.3) (end 144.6 101.6) (width 0.4) (layer B.Cu) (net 11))
 (segment (start 148.94 100.3) (end 147.95 100.3) (width 0.2) (layer F.Cu) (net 2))
 (segment (start 149.86 100.33) (end 148.97 100.33) (width 0.2) (layer F.Cu) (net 2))
 (segment (start 148.97 100.33) (end 148.94 100.3) (width 0.2) (layer F.Cu) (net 2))
 (segment (start 149.86 101.6) (end 147.95 101.6) (width 0.2) (layer F.Cu) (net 4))
 (segment (start 149 102.9) (end 147.95 102.9) (width 0.2) (layer F.Cu) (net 6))
 (segment (start 149.86 102.87) (end 149.03 102.87) (width 0.2) (layer F.Cu) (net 6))
 (segment (start 149.03 102.87) (end 149 102.9) (width 0.2) (layer F.Cu) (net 6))
 (segment (start 148.98 104.2) (end 147.95 104.2) (width 0.2) (layer F.Cu) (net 8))
 (segment (start 149.86 104.14) (end 149.04 104.14) (width 0.2) (layer F.Cu) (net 8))
 (segment (start 149.04 104.14) (end 148.98 104.2) (width 0.2) (layer F.Cu) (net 8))
 (segment (start 149.86 105.41) (end 149.09 105.41) (width 0.2) (layer F.Cu) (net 10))
 (segment (start 149 105.5) (end 147.95 105.5) (width 0.2) (layer F.Cu) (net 10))
 (segment (start 149.09 105.41) (end 149 105.5) (width 0.2) (layer F.Cu) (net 10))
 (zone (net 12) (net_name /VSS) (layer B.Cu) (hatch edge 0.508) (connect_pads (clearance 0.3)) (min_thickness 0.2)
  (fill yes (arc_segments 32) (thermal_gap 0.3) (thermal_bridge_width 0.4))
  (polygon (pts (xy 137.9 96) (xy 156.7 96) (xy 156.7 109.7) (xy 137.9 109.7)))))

